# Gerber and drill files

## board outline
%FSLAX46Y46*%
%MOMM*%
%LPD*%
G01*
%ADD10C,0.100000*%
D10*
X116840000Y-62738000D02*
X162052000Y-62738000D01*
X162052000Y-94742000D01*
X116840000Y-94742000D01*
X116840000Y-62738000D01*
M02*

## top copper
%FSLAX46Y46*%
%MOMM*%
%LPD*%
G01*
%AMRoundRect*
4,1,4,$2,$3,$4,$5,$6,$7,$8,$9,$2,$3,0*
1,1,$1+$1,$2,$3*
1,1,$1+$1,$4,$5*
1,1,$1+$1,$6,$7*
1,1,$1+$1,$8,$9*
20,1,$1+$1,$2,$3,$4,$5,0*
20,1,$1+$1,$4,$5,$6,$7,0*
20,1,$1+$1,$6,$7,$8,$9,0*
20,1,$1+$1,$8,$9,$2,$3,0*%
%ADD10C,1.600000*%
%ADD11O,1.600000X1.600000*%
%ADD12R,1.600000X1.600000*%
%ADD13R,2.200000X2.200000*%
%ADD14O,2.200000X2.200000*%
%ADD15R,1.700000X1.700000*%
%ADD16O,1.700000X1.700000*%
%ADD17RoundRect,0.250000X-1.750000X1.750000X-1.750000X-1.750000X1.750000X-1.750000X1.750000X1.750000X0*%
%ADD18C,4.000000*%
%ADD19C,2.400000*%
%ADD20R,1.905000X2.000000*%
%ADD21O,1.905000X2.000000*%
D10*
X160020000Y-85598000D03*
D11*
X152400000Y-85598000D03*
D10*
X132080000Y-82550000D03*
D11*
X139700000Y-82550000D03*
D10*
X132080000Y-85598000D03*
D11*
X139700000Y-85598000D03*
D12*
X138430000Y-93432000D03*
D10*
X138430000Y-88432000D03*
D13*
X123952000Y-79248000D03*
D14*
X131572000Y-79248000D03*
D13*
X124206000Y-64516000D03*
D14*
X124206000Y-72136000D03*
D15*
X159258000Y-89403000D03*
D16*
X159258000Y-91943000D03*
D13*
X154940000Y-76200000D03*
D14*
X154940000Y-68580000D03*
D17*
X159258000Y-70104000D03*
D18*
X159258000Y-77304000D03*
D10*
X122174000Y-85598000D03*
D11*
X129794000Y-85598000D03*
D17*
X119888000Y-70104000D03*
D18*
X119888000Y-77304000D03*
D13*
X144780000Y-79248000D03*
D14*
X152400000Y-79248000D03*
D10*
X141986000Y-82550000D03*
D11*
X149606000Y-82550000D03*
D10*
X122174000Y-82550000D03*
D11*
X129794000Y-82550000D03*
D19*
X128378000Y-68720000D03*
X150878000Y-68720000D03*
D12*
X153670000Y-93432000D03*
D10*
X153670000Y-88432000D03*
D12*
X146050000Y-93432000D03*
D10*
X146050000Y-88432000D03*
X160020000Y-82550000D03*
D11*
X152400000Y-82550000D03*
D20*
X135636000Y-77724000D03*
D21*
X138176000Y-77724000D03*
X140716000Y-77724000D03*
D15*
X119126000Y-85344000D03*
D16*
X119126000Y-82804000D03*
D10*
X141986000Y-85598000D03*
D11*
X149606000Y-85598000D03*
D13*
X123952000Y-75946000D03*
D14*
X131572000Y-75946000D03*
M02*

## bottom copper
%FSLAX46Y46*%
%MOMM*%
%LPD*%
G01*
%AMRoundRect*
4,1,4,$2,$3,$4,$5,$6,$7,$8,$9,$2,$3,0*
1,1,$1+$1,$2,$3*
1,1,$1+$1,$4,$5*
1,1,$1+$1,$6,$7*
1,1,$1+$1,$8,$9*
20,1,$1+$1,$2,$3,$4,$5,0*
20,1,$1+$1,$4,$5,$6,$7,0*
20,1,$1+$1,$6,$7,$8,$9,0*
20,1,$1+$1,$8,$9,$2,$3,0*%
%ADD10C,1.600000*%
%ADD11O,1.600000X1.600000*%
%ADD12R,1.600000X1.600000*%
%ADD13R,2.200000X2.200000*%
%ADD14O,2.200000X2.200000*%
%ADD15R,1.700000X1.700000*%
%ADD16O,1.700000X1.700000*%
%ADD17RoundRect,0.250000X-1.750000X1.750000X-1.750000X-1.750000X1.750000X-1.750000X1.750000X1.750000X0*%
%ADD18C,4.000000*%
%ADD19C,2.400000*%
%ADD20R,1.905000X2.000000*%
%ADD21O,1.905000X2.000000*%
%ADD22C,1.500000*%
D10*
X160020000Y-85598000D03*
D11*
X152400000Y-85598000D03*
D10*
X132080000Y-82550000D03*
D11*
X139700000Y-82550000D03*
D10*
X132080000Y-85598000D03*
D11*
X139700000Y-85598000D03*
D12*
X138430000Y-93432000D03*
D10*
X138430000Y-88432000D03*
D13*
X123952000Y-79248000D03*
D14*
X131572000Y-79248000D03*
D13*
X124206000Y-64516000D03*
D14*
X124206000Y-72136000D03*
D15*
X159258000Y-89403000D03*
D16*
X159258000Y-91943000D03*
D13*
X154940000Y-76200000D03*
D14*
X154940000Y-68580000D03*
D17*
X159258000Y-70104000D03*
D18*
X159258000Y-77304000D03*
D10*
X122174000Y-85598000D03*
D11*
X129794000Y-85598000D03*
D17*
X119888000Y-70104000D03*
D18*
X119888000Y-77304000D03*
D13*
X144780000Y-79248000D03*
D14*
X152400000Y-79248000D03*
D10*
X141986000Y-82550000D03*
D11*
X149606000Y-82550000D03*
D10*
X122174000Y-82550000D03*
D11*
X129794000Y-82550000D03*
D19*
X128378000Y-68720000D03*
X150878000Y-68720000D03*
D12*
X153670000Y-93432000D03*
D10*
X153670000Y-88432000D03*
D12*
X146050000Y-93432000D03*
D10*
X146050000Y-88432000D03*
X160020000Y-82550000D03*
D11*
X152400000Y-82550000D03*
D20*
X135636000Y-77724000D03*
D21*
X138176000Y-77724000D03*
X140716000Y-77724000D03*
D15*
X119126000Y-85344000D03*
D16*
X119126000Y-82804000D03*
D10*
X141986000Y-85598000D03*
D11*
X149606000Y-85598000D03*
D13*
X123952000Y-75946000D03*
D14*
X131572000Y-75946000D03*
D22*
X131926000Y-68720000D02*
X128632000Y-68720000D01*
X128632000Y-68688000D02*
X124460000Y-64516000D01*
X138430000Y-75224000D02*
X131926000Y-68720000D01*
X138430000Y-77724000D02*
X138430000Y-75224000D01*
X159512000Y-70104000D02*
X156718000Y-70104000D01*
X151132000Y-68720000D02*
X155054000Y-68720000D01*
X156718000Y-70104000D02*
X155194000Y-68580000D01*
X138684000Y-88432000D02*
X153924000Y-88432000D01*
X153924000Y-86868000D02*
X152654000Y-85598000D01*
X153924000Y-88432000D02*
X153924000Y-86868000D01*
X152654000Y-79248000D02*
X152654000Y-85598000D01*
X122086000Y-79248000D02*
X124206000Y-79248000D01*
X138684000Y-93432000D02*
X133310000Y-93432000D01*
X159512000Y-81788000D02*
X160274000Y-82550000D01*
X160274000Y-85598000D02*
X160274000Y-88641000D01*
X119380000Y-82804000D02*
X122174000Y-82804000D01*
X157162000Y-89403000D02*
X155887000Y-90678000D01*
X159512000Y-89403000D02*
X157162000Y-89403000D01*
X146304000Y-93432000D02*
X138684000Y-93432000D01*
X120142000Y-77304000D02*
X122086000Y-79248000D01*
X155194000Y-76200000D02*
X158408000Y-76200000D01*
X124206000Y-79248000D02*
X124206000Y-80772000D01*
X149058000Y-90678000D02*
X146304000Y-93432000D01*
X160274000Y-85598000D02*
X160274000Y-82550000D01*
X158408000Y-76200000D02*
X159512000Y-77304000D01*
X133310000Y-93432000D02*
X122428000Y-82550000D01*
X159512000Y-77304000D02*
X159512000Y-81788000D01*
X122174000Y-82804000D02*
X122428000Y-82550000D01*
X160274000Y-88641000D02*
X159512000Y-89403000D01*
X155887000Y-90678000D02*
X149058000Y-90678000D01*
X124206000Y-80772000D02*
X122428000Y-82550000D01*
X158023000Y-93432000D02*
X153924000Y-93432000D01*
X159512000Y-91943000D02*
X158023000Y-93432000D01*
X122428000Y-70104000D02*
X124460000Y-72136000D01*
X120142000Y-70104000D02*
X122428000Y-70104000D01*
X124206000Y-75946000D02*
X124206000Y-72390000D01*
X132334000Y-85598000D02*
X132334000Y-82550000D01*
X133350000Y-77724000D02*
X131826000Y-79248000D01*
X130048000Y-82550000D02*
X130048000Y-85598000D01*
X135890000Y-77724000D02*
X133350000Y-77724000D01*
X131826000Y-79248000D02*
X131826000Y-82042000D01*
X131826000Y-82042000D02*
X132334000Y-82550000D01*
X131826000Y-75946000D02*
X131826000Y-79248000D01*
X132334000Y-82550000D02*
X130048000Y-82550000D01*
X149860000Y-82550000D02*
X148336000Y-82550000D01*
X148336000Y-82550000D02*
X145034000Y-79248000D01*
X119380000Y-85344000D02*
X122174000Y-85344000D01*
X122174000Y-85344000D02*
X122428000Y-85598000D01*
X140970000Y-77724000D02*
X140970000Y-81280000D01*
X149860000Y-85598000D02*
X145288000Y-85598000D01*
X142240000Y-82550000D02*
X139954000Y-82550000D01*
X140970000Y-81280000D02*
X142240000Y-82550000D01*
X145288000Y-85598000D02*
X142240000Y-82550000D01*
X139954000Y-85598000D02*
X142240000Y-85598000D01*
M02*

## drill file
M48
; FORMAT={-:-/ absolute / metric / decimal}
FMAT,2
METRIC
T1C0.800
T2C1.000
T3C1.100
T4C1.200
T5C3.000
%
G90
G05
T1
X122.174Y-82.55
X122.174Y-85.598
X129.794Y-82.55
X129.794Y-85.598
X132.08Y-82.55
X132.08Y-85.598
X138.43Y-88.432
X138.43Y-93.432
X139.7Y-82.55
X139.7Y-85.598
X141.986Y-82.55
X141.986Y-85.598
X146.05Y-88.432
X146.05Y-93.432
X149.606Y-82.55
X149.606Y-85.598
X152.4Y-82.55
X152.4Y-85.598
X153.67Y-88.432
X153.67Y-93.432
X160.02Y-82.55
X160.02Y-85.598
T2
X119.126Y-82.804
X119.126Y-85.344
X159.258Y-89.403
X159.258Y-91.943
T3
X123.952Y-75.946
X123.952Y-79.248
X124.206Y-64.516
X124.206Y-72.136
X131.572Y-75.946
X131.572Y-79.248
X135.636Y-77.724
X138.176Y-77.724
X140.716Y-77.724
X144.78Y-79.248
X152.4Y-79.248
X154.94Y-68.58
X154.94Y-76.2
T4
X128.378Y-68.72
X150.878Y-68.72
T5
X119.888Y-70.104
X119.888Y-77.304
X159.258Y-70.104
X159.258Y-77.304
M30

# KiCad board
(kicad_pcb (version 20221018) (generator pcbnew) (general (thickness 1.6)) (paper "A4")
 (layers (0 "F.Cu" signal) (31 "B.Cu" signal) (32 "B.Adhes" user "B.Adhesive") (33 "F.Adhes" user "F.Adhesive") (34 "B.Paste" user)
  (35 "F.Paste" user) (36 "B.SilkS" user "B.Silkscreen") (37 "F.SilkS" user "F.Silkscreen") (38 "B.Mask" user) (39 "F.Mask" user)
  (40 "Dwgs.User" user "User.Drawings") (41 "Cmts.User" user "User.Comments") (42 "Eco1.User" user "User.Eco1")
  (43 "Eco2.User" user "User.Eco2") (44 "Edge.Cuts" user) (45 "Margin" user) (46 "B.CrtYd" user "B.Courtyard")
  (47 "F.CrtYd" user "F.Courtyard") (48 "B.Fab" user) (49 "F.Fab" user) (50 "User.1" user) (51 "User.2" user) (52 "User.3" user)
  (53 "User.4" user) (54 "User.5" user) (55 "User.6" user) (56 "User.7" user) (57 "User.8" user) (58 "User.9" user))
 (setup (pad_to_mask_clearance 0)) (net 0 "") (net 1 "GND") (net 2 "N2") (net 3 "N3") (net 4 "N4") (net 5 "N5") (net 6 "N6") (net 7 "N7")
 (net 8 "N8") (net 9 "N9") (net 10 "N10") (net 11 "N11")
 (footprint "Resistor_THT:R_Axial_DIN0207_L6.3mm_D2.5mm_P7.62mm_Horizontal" (layer "F.Cu") (at 160.02 85.598 180)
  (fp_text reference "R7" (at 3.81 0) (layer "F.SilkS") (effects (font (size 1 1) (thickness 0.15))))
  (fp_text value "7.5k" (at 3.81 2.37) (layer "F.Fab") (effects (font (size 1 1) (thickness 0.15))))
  (pad "1" thru_hole circle (at 0 0 180) (size 1.6 1.6) (drill 0.8) (layers "*.Cu" "*.Mask") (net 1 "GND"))
  (pad "2" thru_hole oval (at 7.62 0 180) (size 1.6 1.6) (drill 0.8) (layers "*.Cu" "*.Mask") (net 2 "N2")))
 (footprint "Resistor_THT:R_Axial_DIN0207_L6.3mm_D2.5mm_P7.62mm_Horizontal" (layer "F.Cu") (at 132.08 82.55)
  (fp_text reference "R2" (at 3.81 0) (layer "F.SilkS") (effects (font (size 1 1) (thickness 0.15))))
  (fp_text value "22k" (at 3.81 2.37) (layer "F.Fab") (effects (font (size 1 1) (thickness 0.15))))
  (pad "1" thru_hole circle (at 0 0) (size 1.6 1.6) (drill 0.8) (layers "*.Cu" "*.Mask") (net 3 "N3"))
  (pad "2" thru_hole oval (at 7.62 0) (size 1.6 1.6) (drill 0.8) (layers "*.Cu" "*.Mask") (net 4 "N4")))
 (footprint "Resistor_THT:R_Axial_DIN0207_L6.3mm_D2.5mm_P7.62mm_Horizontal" (layer "F.Cu") (at 132.08 85.598)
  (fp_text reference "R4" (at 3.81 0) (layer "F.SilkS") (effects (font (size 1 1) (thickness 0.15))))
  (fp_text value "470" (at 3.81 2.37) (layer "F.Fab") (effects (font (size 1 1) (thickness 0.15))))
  (pad "1" thru_hole circle (at 0 0) (size 1.6 1.6) (drill 0.8) (layers "*.Cu" "*.Mask") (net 3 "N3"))
  (pad "2" thru_hole oval (at 7.62 0) (size 1.6 1.6) (drill 0.8) (layers "*.Cu" "*.Mask") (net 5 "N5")))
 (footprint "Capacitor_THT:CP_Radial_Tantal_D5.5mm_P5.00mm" (layer "F.Cu") (at 138.43 93.432 90)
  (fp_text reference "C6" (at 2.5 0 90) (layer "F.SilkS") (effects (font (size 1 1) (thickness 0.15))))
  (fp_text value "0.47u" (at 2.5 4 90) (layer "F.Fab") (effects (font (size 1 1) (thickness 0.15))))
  (pad "1" thru_hole rect (at 0 0 90) (size 1.6 1.6) (drill 0.8) (layers "*.Cu" "*.Mask") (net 1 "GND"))
  (pad "2" thru_hole circle (at 5 0 90) (size 1.6 1.6) (drill 0.8) (layers "*.Cu" "*.Mask") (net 2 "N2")))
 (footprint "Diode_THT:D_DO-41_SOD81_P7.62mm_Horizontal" (layer "F.Cu") (at 123.952 79.248)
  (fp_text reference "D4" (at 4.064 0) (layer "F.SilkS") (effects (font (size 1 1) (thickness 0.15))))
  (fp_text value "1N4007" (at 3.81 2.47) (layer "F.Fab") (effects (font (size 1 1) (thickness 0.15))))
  (pad "1" thru_hole rect (at 0 0) (size 2.2 2.2) (drill 1.1) (layers "*.Cu" "*.Mask") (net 1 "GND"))
  (pad "2" thru_hole oval (at 7.62 0) (size 2.2 2.2) (drill 1.1) (layers "*.Cu" "*.Mask") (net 3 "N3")))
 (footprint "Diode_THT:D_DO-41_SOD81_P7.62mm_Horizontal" (layer "F.Cu") (at 124.206 64.516 -90)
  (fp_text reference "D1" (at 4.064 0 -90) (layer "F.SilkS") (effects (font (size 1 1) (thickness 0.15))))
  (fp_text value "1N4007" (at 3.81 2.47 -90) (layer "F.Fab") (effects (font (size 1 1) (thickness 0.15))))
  (pad "1" thru_hole rect (at 0 0 270) (size 2.2 2.2) (drill 1.1) (layers "*.Cu" "*.Mask") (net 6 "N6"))
  (pad "2" thru_hole oval (at 7.62 0 270) (size 2.2 2.2) (drill 1.1) (layers "*.Cu" "*.Mask") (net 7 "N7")))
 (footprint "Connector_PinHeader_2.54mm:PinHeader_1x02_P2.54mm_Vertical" (layer "F.Cu") (at 159.258 89.403)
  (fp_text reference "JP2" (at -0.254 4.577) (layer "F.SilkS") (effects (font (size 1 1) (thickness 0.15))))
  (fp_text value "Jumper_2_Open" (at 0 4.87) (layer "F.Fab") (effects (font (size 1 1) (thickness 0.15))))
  (pad "1" thru_hole rect (at 0 0) (size 1.7 1.7) (drill 1) (layers "*.Cu" "*.Mask") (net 1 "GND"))
  (pad "2" thru_hole oval (at 0 2.54) (size 1.7 1.7) (drill 1) (layers "*.Cu" "*.Mask") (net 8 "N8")))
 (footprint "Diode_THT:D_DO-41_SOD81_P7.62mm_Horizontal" (layer "F.Cu") (at 154.94 76.2 90)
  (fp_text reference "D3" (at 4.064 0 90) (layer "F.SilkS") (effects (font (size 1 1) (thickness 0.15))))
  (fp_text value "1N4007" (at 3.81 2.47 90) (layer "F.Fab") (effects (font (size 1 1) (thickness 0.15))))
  (pad "1" thru_hole rect (at 0 0 90) (size 2.2 2.2) (drill 1.1) (layers "*.Cu" "*.Mask") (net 1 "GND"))
  (pad "2" thru_hole oval (at 7.62 0 90) (size 2.2 2.2) (drill 1.1) (layers "*.Cu" "*.Mask") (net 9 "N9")))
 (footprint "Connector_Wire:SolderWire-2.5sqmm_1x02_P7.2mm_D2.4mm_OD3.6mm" (layer "F.Cu") (at 159.258 70.104 -90)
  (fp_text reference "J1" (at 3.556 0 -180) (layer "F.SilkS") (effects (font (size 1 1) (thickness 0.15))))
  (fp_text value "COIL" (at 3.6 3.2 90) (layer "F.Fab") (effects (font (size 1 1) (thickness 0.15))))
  (pad "1" thru_hole roundrect (at 0 0 270) (size 4 4) (drill 3) (layers "*.Cu" "*.Mask") (roundrect_rratio 0.0625) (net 9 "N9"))
  (pad "2" thru_hole circle (at 7.2 0 270) (size 4 4) (drill 3) (layers "*.Cu" "*.Mask") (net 1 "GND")))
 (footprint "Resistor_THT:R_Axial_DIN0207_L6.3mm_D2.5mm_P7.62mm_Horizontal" (layer "F.Cu") (at 122.174 85.598)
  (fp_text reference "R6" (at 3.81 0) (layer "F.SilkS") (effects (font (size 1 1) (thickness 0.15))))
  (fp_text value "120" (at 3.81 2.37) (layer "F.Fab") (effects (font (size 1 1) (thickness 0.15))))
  (pad "1" thru_hole circle (at 0 0) (size 1.6 1.6) (drill 0.8) (layers "*.Cu" "*.Mask") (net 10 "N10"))
  (pad "2" thru_hole oval (at 7.62 0) (size 1.6 1.6) (drill 0.8) (layers "*.Cu" "*.Mask") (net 3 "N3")))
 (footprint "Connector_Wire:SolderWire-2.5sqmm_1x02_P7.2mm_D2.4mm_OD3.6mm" (layer "F.Cu") (at 119.888 70.104 -90)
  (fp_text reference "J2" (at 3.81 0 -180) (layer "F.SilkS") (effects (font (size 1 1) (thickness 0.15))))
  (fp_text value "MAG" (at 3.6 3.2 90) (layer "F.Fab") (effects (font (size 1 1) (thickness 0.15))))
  (pad "1" thru_hole roundrect (at 0 0 270) (size 4 4) (drill 3) (layers "*.Cu" "*.Mask") (roundrect_rratio 0.0625) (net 7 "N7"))
  (pad "2" thru_hole circle (at 7.2 0 270) (size 4 4) (drill 3) (layers "*.Cu" "*.Mask") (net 1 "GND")))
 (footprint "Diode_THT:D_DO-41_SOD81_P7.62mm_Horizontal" (layer "F.Cu") (at 144.78 79.248)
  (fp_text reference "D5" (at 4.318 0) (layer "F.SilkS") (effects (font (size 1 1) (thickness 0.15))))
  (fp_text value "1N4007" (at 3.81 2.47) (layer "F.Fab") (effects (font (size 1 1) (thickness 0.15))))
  (pad "1" thru_hole rect (at 0 0) (size 2.2 2.2) (drill 1.1) (layers "*.Cu" "*.Mask") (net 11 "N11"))
  (pad "2" thru_hole oval (at 7.62 0) (size 2.2 2.2) (drill 1.1) (layers "*.Cu" "*.Mask") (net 2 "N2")))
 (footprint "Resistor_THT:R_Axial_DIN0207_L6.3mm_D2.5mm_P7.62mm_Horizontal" (layer "F.Cu") (at 141.986 82.55)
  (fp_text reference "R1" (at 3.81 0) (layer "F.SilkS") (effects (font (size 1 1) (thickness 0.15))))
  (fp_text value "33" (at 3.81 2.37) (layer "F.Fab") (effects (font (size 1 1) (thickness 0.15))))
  (pad "1" thru_hole circle (at 0 0) (size 1.6 1.6) (drill 0.8) (layers "*.Cu" "*.Mask") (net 4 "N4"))
  (pad "2" thru_hole oval (at 7.62 0) (size 1.6 1.6) (drill 0.8) (layers "*.Cu" "*.Mask") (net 11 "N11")))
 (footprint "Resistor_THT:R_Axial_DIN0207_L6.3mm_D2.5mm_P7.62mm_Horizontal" (layer "F.Cu") (at 122.174 82.55)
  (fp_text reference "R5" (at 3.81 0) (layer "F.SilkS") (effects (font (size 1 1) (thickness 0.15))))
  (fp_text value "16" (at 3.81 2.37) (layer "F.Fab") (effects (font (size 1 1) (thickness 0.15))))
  (pad "1" thru_hole circle (at 0 0) (size 1.6 1.6) (drill 0.8) (layers "*.Cu" "*.Mask") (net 1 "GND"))
  (pad "2" thru_hole oval (at 7.62 0) (size 1.6 1.6) (drill 0.8) (layers "*.Cu" "*.Mask") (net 3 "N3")))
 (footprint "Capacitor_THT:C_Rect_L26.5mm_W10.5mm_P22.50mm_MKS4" (layer "F.Cu") (at 128.378 68.72)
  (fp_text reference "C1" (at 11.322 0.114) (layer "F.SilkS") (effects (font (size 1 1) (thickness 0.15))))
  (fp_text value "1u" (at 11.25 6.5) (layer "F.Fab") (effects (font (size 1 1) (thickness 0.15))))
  (pad "1" thru_hole circle (at 0 0) (size 2.4 2.4) (drill 1.2) (layers "*.Cu" "*.Mask") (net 6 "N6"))
  (pad "2" thru_hole circle (at 22.5 0) (size 2.4 2.4) (drill 1.2) (layers "*.Cu" "*.Mask") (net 9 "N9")))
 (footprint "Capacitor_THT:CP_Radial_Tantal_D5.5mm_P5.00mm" (layer "F.Cu") (at 153.67 93.432 90)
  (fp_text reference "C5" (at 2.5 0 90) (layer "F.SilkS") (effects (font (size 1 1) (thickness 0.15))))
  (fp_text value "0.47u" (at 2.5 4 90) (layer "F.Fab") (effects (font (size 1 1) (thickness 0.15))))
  (pad "1" thru_hole rect (at 0 0 90) (size 1.6 1.6) (drill 0.8) (layers "*.Cu" "*.Mask") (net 8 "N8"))
  (pad "2" thru_hole circle (at 5 0 90) (size 1.6 1.6) (drill 0.8) (layers "*.Cu" "*.Mask") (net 2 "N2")))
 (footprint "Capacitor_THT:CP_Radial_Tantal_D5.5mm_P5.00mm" (layer "F.Cu") (at 146.05 93.432 90)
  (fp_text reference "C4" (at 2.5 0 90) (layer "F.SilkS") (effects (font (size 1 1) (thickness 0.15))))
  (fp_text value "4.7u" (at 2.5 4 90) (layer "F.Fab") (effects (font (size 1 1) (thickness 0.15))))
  (pad "1" thru_hole rect (at 0 0 90) (size 1.6 1.6) (drill 0.8) (layers "*.Cu" "*.Mask") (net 1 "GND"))
  (pad "2" thru_hole circle (at 5 0 90) (size 1.6 1.6) (drill 0.8) (layers "*.Cu" "*.Mask") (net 2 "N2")))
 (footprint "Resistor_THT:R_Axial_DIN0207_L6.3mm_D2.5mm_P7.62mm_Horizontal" (layer "F.Cu") (at 160.02 82.55 180)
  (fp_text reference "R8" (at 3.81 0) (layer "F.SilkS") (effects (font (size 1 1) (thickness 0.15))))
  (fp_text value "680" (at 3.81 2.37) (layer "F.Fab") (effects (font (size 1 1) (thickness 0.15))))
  (pad "1" thru_hole circle (at 0 0 180) (size 1.6 1.6) (drill 0.8) (layers "*.Cu" "*.Mask") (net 1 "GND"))
  (pad "2" thru_hole oval (at 7.62 0 180) (size 1.6 1.6) (drill 0.8) (layers "*.Cu" "*.Mask") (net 2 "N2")))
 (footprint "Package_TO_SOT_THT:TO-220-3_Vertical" (layer "F.Cu") (at 135.636 77.724)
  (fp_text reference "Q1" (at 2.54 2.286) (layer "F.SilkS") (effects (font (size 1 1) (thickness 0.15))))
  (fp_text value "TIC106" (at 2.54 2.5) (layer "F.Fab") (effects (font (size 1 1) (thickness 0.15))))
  (pad "1" thru_hole rect (at 0 0) (size 1.905 2) (drill 1.1) (layers "*.Cu" "*.Mask") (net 3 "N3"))
  (pad "2" thru_hole oval (at 2.54 0) (size 1.905 2) (drill 1.1) (layers "*.Cu" "*.Mask") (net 6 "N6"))
  (pad "3" thru_hole oval (at 5.08 0) (size 1.905 2) (drill 1.1) (layers "*.Cu" "*.Mask") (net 4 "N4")))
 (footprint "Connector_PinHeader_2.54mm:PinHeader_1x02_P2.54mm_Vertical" (layer "F.Cu") (at 119.126 85.344 180)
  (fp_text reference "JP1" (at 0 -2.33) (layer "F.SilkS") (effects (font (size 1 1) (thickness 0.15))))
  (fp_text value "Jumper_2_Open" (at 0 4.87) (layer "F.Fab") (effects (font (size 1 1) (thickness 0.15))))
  (pad "1" thru_hole rect (at 0 0 180) (size 1.7 1.7) (drill 1) (layers "*.Cu" "*.Mask") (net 10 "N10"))
  (pad "2" thru_hole oval (at 0 2.54 180) (size 1.7 1.7) (drill 1) (layers "*.Cu" "*.Mask") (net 1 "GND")))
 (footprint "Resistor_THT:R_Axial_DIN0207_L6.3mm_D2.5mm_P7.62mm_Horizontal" (layer "F.Cu") (at 141.986 85.598)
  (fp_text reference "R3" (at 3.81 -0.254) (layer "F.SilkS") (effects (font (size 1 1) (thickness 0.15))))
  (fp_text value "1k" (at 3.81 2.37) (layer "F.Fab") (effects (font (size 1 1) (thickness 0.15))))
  (pad "1" thru_hole circle (at 0 0) (size 1.6 1.6) (drill 0.8) (layers "*.Cu" "*.Mask") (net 5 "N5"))
  (pad "2" thru_hole oval (at 7.62 0) (size 1.6 1.6) (drill 0.8) (layers "*.Cu" "*.Mask") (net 4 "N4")))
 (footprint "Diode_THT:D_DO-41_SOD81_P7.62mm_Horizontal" (layer "F.Cu") (at 123.952 75.946)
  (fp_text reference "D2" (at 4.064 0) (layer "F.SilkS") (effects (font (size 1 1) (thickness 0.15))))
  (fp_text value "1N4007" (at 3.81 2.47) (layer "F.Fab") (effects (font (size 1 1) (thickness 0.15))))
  (pad "1" thru_hole rect (at 0 0) (size 2.2 2.2) (drill 1.1) (layers "*.Cu" "*.Mask") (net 7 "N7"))
  (pad "2" thru_hole oval (at 7.62 0) (size 2.2 2.2) (drill 1.1) (layers "*.Cu" "*.Mask") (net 3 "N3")))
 (gr_rect (start 116.84 62.738) (end 162.052 94.742) (stroke (width 0.1) (type default)) (fill none) (layer "Edge.Cuts"))
 (segment (start 131.926 68.72) (end 128.632 68.72) (width 1.5) (layer "B.Cu") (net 6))
 (segment (start 128.632 68.688) (end 124.46 64.516) (width 1.5) (layer "B.Cu") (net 6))
 (segment (start 138.43 75.224) (end 131.926 68.72) (width 1.5) (layer "B.Cu") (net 6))
 (segment (start 138.43 77.724) (end 138.43 75.224) (width 1.5) (layer "B.Cu") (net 6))
 (segment (start 159.512 70.104) (end 156.718 70.104) (width 1.5) (layer "B.Cu") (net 9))
 (segment (start 151.132 68.72) (end 155.054 68.72) (width 1.5) (layer "B.Cu") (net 9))
 (segment (start 156.718 70.104) (end 155.194 68.58) (width 1.5) (layer "B.Cu") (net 9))
 (segment (start 138.684 88.432) (end 153.924 88.432) (width 1.5) (layer "B.Cu") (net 2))
 (segment (start 153.924 86.868) (end 152.654 85.598) (width 1.5) (layer "B.Cu") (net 2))
 (segment (start 153.924 88.432) (end 153.924 86.868) (width 1.5) (layer "B.Cu") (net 2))
 (segment (start 152.654 79.248) (end 152.654 85.598) (width 1.5) (layer "B.Cu") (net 2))
 (segment (start 122.086 79.248) (end 124.206 79.248) (width 1.5) (layer "B.Cu") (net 1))
 (segment (start 138.684 93.432) (end 133.31 93.432) (width 1.5) (layer "B.Cu") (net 1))
 (segment (start 159.512 81.788) (end 160.274 82.55) (width 1.5) (layer "B.Cu") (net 1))
 (segment (start 160.274 85.598) (end 160.274 88.641) (width 1.5) (layer "B.Cu") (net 1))
 (segment (start 119.38 82.804) (end 122.174 82.804) (width 1.5) (layer "B.Cu") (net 1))
 (segment (start 157.162 89.403) (end 155.887 90.678) (width 1.5) (layer "B.Cu") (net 1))
 (segment (start 159.512 89.403) (end 157.162 89.403) (width 1.5) (layer "B.Cu") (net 1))
 (segment (start 146.304 93.432) (end 138.684 93.432) (width 1.5) (layer "B.Cu") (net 1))
 (segment (start 120.142 77.304) (end 122.086 79.248) (width 1.5) (layer "B.Cu") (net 1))
 (segment (start 155.194 76.2) (end 158.408 76.2) (width 1.5) (layer "B.Cu") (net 1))
 (segment (start 124.206 79.248) (end 124.206 80.772) (width 1.5) (layer "B.Cu") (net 1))
 (segment (start 149.058 90.678) (end 146.304 93.432) (width 1.5) (layer "B.Cu") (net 1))
 (segment (start 160.274 85.598) (end 160.274 82.55) (width 1.5) (layer "B.Cu") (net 1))
 (segment (start 158.408 76.2) (end 159.512 77.304) (width 1.5) (layer "B.Cu") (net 1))
 (segment (start 133.31 93.432) (end 122.428 82.55) (width 1.5) (layer "B.Cu") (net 1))
 (segment (start 159.512 77.304) (end 159.512 81.788) (width 1.5) (layer "B.Cu") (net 1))
 (segment (start 122.174 82.804) (end 122.428 82.55) (width 1.5) (layer "B.Cu") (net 1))
 (segment (start 160.274 88.641) (end 159.512 89.403) (width 1.5) (layer "B.Cu") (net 1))
 (segment (start 155.887 90.678) (end 149.058 90.678) (width 1.5) (layer "B.Cu") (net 1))
 (segment (start 124.206 80.772) (end 122.428 82.55) (width 1.5) (layer "B.Cu") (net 1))
 (segment (start 158.023 93.432) (end 153.924 93.432) (width 1.5) (layer "B.Cu") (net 8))
 (segment (start 159.512 91.943) (end 158.023 93.432) (width 1.5) (layer "B.Cu") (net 8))
 (segment (start 122.428 70.104) (end 124.46 72.136) (width 1.5) (layer "B.Cu") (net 7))
 (segment (start 120.142 70.104) (end 122.428 70.104) (width 1.5) (layer "B.Cu") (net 7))
 (segment (start 124.206 75.946) (end 124.206 72.39) (width 1.5) (layer "B.Cu") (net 7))
 (segment (start 132.334 85.598) (end 132.334 82.55) (width 1.5) (layer "B.Cu") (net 3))
 (segment (start 133.35 77.724) (end 131.826 79.248) (width 1.5) (layer "B.Cu") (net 3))
 (segment (start 130.048 82.55) (end 130.048 85.598) (width 1.5) (layer "B.Cu") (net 3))
 (segment (start 135.89 77.724) (end 133.35 77.724) (width 1.5) (layer "B.Cu") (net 3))
 (segment (start 131.826 79.248) (end 131.826 82.042) (width 1.5) (layer "B.Cu") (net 3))
 (segment (start 131.826 82.042) (end 132.334 82.55) (width 1.5) (layer "B.Cu") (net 3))
 (segment (start 131.826 75.946) (end 131.826 79.248) (width 1.5) (layer "B.Cu") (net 3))
 (segment (start 132.334 82.55) (end 130.048 82.55) (width 1.5) (layer "B.Cu") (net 3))
 (segment (start 149.86 82.55) (end 148.336 82.55) (width 1.5) (layer "B.Cu") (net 11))
 (segment (start 148.336 82.55) (end 145.034 79.248) (width 1.5) (layer "B.Cu") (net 11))
 (segment (start 119.38 85.344) (end 122.174 85.344) (width 1.5) (layer "B.Cu") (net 10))
 (segment (start 122.174 85.344) (end 122.428 85.598) (width 1.5) (layer "B.Cu") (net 10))
 (segment (start 140.97 77.724) (end 140.97 81.28) (width 1.5) (layer "B.Cu") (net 4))
 (segment (start 149.86 85.598) (end 145.288 85.598) (width 1.5) (layer "B.Cu") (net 4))
 (segment (start 142.24 82.55) (end 139.954 82.55) (width 1.5) (layer "B.Cu") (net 4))
 (segment (start 140.97 81.28) (end 142.24 82.55) (width 1.5) (layer "B.Cu") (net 4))
 (segment (start 145.288 85.598) (end 142.24 82.55) (width 1.5) (layer "B.Cu") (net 4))
 (segment (start 139.954 85.598) (end 142.24 85.598) (width 1.5) (layer "B.Cu") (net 5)))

